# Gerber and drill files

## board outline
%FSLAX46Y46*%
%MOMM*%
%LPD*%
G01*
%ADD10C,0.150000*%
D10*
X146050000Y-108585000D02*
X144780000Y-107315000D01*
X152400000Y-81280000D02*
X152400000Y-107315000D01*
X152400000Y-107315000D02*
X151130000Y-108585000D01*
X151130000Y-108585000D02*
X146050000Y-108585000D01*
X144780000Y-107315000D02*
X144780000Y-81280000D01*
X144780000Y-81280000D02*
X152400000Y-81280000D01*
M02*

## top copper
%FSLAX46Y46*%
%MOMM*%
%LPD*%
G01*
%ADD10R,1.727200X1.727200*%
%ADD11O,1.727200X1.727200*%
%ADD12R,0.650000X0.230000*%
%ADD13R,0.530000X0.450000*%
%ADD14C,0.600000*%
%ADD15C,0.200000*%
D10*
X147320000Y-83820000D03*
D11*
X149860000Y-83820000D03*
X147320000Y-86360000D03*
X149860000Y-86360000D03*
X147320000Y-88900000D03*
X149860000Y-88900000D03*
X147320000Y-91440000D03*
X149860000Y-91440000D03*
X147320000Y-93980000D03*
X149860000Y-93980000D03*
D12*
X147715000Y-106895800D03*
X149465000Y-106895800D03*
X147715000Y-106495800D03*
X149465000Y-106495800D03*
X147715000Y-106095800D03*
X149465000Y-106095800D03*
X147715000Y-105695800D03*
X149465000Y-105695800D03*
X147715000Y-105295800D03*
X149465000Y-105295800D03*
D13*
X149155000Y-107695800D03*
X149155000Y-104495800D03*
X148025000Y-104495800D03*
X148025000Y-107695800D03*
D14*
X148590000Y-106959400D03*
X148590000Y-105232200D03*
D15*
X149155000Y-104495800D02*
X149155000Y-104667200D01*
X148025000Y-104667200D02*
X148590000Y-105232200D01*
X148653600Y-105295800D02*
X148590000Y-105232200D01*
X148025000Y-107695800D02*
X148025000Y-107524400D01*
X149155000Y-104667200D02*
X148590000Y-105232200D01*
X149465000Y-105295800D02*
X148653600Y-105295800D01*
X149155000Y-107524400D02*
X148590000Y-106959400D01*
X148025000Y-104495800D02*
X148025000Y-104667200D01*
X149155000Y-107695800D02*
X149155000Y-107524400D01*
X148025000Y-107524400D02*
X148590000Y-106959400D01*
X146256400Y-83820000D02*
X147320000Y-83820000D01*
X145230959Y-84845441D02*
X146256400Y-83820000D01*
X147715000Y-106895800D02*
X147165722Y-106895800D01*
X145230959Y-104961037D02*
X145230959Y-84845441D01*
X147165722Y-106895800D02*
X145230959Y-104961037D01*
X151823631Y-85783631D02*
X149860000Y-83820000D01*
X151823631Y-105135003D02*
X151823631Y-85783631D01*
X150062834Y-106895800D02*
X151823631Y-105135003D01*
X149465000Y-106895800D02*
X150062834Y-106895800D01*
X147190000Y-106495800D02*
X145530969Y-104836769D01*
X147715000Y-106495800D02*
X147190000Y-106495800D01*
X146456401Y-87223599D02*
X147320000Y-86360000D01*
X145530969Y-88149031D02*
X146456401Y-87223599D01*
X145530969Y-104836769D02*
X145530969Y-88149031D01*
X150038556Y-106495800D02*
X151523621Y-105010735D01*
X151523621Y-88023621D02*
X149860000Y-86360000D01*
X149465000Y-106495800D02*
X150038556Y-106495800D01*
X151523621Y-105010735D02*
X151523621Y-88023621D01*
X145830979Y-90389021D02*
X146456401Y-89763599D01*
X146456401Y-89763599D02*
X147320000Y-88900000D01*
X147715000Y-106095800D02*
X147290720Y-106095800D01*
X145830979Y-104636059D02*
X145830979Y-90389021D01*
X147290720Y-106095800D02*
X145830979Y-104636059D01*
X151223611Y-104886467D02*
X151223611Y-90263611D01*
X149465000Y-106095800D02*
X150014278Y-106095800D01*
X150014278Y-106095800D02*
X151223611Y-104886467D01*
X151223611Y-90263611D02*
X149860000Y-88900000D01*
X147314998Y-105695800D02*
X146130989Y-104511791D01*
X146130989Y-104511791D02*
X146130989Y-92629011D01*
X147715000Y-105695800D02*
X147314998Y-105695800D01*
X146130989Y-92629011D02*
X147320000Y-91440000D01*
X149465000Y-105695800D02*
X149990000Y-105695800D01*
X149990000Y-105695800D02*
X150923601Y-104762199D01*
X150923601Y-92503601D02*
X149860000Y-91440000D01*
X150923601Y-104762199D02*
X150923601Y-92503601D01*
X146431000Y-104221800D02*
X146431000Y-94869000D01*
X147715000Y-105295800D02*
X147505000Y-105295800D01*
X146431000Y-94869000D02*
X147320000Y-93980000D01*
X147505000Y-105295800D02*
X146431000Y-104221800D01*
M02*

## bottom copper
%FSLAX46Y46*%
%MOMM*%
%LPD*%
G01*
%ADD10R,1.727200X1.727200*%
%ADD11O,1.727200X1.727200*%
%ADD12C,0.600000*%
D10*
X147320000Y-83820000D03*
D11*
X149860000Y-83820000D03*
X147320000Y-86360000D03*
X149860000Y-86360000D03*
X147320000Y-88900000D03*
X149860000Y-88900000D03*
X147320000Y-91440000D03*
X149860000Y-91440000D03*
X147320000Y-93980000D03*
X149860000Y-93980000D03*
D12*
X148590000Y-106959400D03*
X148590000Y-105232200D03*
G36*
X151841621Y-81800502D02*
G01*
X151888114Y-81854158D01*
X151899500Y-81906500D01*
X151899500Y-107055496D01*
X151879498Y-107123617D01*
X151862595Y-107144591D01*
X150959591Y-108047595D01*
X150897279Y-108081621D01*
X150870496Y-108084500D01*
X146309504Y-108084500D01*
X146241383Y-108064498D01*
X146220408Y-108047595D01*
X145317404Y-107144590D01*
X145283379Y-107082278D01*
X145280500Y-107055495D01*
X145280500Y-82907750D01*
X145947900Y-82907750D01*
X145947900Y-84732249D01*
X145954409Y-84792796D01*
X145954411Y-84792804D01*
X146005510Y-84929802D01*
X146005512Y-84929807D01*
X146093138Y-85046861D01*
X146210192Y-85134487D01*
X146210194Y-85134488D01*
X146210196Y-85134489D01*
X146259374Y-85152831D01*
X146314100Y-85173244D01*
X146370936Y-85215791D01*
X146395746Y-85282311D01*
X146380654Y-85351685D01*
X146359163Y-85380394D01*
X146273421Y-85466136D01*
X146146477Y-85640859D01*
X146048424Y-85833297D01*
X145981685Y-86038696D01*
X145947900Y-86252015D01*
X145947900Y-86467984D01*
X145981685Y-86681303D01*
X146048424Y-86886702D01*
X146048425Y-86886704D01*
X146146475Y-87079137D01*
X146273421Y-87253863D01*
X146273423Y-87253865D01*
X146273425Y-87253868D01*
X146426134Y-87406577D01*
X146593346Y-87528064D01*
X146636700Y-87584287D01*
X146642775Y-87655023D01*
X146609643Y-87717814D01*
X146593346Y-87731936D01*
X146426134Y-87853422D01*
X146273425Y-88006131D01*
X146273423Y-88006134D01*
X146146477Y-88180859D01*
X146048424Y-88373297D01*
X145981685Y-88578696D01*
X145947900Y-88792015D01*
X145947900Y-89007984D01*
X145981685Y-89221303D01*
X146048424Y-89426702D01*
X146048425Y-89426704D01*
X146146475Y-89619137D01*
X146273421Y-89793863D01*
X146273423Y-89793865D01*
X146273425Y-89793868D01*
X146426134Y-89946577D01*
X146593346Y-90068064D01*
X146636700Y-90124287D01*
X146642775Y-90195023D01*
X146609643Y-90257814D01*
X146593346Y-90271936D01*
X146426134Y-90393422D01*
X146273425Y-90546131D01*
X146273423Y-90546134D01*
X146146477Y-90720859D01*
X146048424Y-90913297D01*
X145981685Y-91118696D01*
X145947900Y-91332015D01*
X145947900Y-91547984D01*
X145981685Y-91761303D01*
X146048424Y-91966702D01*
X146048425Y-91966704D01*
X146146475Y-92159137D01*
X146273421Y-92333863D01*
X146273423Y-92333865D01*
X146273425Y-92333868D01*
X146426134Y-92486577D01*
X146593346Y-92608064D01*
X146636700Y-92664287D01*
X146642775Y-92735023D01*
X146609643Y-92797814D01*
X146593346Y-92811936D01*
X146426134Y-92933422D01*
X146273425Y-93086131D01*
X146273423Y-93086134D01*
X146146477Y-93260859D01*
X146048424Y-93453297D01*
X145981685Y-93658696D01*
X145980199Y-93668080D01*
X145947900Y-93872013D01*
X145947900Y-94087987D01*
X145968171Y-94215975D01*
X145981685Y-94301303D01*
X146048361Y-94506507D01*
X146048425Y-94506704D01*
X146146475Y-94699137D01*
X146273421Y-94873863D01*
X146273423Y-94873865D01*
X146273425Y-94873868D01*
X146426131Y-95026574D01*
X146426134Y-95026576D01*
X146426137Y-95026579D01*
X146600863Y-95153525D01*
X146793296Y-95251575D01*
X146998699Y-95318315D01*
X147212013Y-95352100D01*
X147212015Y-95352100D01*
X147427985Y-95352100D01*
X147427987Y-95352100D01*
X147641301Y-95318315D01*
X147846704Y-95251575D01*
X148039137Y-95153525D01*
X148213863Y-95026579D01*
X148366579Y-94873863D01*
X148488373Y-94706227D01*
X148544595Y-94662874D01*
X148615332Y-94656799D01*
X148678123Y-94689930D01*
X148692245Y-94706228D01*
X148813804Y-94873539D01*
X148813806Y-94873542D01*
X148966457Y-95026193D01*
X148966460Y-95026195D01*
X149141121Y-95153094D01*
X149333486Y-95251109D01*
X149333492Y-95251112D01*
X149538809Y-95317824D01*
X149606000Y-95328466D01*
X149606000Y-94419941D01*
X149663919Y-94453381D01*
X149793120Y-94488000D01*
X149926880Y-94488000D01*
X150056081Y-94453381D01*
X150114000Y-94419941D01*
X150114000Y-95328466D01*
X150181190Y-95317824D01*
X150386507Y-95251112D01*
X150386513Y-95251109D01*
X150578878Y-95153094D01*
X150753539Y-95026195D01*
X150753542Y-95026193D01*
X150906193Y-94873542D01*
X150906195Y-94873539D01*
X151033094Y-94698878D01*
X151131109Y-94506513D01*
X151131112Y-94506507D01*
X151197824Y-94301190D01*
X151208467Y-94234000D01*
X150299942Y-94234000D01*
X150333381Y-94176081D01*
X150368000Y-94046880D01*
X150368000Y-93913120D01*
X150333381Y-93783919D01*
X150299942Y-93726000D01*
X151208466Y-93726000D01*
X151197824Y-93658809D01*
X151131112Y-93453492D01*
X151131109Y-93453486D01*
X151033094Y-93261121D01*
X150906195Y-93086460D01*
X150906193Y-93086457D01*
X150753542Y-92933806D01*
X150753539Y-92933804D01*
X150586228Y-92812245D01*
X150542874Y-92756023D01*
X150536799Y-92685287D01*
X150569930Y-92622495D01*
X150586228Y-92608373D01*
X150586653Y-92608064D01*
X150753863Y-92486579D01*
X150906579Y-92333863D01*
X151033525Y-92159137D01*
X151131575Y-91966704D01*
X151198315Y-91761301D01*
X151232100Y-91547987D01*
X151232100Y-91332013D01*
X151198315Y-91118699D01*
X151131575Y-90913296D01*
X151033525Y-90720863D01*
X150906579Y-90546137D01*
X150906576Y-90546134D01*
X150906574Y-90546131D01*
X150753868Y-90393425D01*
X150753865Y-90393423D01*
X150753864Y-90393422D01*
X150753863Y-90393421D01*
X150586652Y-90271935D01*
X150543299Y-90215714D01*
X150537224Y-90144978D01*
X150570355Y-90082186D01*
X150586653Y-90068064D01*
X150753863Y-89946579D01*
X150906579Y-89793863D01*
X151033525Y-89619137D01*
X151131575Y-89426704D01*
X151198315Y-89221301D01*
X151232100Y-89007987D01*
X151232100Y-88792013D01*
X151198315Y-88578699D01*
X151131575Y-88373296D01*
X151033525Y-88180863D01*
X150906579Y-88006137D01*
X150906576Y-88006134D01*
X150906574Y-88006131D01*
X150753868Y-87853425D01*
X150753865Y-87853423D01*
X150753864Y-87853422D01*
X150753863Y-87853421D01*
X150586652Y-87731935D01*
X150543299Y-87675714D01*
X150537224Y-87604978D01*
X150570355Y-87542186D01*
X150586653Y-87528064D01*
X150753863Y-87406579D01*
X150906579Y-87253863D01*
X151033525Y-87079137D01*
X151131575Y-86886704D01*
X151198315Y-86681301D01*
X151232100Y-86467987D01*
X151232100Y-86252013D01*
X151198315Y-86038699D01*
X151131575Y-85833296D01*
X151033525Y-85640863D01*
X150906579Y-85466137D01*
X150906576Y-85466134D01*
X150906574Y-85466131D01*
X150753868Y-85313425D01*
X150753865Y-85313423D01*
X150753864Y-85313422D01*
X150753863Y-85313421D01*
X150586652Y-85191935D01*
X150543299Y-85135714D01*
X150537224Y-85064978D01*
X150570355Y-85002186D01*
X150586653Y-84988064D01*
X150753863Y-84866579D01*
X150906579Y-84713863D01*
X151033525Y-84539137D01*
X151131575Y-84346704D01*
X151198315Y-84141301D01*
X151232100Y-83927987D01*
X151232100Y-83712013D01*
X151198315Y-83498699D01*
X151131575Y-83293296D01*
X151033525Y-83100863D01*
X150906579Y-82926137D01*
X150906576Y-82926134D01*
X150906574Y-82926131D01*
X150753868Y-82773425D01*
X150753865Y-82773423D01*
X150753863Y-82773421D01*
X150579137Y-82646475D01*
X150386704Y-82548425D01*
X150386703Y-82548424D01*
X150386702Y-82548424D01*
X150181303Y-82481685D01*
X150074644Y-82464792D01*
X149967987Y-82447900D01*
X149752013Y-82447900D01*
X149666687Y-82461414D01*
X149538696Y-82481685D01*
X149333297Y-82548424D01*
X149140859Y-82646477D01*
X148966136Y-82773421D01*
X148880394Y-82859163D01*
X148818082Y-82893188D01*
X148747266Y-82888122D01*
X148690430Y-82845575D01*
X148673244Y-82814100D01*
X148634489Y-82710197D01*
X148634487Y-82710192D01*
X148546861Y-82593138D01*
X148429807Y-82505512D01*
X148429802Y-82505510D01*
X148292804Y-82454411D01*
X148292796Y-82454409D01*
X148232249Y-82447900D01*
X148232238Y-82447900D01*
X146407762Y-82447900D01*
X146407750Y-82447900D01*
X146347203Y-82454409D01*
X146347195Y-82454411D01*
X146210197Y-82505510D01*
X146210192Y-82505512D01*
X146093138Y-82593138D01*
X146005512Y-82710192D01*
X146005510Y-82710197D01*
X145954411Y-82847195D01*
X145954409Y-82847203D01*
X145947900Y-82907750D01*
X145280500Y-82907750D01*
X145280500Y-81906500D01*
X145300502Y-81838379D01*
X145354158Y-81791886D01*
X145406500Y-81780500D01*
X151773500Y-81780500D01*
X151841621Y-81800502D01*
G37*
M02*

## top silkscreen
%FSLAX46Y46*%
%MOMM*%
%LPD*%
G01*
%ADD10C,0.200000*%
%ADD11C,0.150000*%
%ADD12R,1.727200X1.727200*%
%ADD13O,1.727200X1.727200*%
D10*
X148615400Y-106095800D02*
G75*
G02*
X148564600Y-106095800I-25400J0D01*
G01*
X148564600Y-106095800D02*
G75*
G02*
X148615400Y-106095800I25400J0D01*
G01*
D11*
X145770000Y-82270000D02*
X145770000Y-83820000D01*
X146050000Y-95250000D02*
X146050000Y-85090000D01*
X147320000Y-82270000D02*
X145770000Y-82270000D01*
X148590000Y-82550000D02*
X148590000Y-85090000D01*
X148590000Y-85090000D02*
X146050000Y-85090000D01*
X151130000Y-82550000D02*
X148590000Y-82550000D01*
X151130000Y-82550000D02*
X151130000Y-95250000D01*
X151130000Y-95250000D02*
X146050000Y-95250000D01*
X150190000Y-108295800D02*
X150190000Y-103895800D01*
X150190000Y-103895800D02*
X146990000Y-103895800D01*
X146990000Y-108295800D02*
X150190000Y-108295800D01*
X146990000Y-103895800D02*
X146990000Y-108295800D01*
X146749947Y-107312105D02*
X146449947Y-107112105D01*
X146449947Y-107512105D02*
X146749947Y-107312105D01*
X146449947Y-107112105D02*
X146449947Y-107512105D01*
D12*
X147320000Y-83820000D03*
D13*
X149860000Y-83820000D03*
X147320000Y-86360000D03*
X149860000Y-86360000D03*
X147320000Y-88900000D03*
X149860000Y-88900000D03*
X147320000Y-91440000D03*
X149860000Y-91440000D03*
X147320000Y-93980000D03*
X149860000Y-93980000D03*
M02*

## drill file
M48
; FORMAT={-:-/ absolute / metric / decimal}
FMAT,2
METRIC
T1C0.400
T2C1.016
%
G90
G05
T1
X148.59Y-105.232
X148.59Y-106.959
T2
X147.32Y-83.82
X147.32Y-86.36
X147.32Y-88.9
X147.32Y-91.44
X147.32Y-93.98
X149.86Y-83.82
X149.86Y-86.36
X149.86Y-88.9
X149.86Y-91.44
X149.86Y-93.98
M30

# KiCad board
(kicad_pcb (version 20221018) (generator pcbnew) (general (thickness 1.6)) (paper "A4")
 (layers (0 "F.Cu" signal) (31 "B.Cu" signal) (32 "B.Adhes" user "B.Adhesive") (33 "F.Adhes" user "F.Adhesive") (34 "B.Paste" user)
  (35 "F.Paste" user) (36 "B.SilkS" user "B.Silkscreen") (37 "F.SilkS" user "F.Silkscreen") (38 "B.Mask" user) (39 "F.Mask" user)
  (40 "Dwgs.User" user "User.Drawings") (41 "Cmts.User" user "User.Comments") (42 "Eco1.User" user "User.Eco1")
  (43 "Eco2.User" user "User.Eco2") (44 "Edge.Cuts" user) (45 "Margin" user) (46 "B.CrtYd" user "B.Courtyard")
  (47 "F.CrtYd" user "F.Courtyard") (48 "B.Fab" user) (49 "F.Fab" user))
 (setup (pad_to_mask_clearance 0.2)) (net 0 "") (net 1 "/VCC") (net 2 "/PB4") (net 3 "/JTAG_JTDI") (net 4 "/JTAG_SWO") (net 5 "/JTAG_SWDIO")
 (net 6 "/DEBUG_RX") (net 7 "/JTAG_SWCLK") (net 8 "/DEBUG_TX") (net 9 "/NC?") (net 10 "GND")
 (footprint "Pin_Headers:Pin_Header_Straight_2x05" (layer "F.Cu") (at 147.32 83.82)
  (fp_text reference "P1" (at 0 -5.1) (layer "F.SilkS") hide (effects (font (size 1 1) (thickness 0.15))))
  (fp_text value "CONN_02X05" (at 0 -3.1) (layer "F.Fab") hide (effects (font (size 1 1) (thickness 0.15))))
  (fp_line (start -1.55 -1.55) (end -1.55 0) (stroke (width 0.15) (type solid)) (layer "F.SilkS"))
  (fp_line (start -1.27 11.43) (end -1.27 1.27) (stroke (width 0.15) (type solid)) (layer "F.SilkS"))
  (fp_line (start 0 -1.55) (end -1.55 -1.55) (stroke (width 0.15) (type solid)) (layer "F.SilkS"))
  (fp_line (start 1.27 -1.27) (end 1.27 1.27) (stroke (width 0.15) (type solid)) (layer "F.SilkS"))
  (fp_line (start 1.27 1.27) (end -1.27 1.27) (stroke (width 0.15) (type solid)) (layer "F.SilkS"))
  (fp_line (start 3.81 -1.27) (end 1.27 -1.27) (stroke (width 0.15) (type solid)) (layer "F.SilkS"))
  (fp_line (start 3.81 -1.27) (end 3.81 11.43) (stroke (width 0.15) (type solid)) (layer "F.SilkS"))
  (fp_line (start 3.81 11.43) (end -1.27 11.43) (stroke (width 0.15) (type solid)) (layer "F.SilkS"))
  (pad "1" thru_hole rect (at 0 0) (size 1.7272 1.7272) (drill 1.016) (layers "*.Cu" "*.Mask" "F.SilkS") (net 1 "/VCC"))
  (pad "2" thru_hole oval (at 2.54 0) (size 1.7272 1.7272) (drill 1.016) (layers "*.Cu" "*.Mask" "F.SilkS") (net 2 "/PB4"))
  (pad "3" thru_hole oval (at 0 2.54) (size 1.7272 1.7272) (drill 1.016) (layers "*.Cu" "*.Mask" "F.SilkS") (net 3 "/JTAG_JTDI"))
  (pad "4" thru_hole oval (at 2.54 2.54) (size 1.7272 1.7272) (drill 1.016) (layers "*.Cu" "*.Mask" "F.SilkS") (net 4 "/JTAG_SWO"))
  (pad "5" thru_hole oval (at 0 5.08) (size 1.7272 1.7272) (drill 1.016) (layers "*.Cu" "*.Mask" "F.SilkS") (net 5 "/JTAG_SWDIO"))
  (pad "6" thru_hole oval (at 2.54 5.08) (size 1.7272 1.7272) (drill 1.016) (layers "*.Cu" "*.Mask" "F.SilkS") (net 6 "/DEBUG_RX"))
  (pad "7" thru_hole oval (at 0 7.62) (size 1.7272 1.7272) (drill 1.016) (layers "*.Cu" "*.Mask" "F.SilkS") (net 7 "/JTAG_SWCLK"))
  (pad "8" thru_hole oval (at 2.54 7.62) (size 1.7272 1.7272) (drill 1.016) (layers "*.Cu" "*.Mask" "F.SilkS") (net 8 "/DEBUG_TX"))
  (pad "9" thru_hole oval (at 0 10.16) (size 1.7272 1.7272) (drill 1.016) (layers "*.Cu" "*.Mask" "F.SilkS") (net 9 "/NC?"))
  (pad "10" thru_hole oval (at 2.54 10.16) (size 1.7272 1.7272) (drill 1.016) (layers "*.Cu" "*.Mask" "F.SilkS") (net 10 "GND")))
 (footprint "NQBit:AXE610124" (layer "F.Cu") (at 148.59 106.0958 180)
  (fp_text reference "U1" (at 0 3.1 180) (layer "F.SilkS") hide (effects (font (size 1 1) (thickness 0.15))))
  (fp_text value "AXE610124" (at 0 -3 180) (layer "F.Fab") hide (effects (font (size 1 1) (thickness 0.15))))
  (fp_line (start -1.6 -2.2) (end -1.6 2.2) (stroke (width 0.15) (type solid)) (layer "F.SilkS"))
  (fp_line (start -1.6 2.2) (end 1.6 2.2) (stroke (width 0.15) (type solid)) (layer "F.SilkS"))
  (fp_line (start 1.6 -2.2) (end -1.6 -2.2) (stroke (width 0.15) (type solid)) (layer "F.SilkS"))
  (fp_line (start 1.6 2.2) (end 1.6 -2.2) (stroke (width 0.15) (type solid)) (layer "F.SilkS"))
  (fp_line (start 1.840053 -1.216305) (end 2.140053 -1.016305) (stroke (width 0.15) (type solid)) (layer "F.SilkS"))
  (fp_line (start 2.140053 -1.416305) (end 1.840053 -1.216305) (stroke (width 0.15) (type solid)) (layer "F.SilkS"))
  (fp_line (start 2.140053 -1.016305) (end 2.140053 -1.416305) (stroke (width 0.15) (type solid)) (layer "F.SilkS"))
  (pad "1" smd rect (at 0.875 -0.8 180) (size 0.65 0.23) (layers "F.Cu" "F.Paste" "F.Mask") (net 1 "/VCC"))
  (pad "2" smd rect (at -0.875 -0.8 180) (size 0.65 0.23) (layers "F.Cu" "F.Paste" "F.Mask") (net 2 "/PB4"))
  (pad "3" smd rect (at 0.875 -0.4 180) (size 0.65 0.23) (layers "F.Cu" "F.Paste" "F.Mask") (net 3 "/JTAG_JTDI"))
  (pad "4" smd rect (at -0.875 -0.4 180) (size 0.65 0.23) (layers "F.Cu" "F.Paste" "F.Mask") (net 4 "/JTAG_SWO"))
  (pad "5" smd rect (at 0.875 0 180) (size 0.65 0.23) (layers "F.Cu" "F.Paste" "F.Mask") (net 5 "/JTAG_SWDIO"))
  (pad "6" smd rect (at -0.875 0 180) (size 0.65 0.23) (layers "F.Cu" "F.Paste" "F.Mask") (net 6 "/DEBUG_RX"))
  (pad "7" smd rect (at 0.875 0.4 180) (size 0.65 0.23) (layers "F.Cu" "F.Paste" "F.Mask") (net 7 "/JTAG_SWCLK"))
  (pad "8" smd rect (at -0.875 0.4 180) (size 0.65 0.23) (layers "F.Cu" "F.Paste" "F.Mask") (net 8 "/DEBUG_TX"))
  (pad "9" smd rect (at 0.875 0.8 180) (size 0.65 0.23) (layers "F.Cu" "F.Paste" "F.Mask") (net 9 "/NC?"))
  (pad "10" smd rect (at -0.875 0.8 180) (size 0.65 0.23) (layers "F.Cu" "F.Paste" "F.Mask") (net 10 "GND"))
  (pad "P1" smd rect (at -0.565 -1.6 180) (size 0.53 0.45) (layers "F.Cu" "F.Paste" "F.Mask") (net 10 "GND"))
  (pad "P2" smd rect (at -0.565 1.6 180) (size 0.53 0.45) (layers "F.Cu" "F.Paste" "F.Mask") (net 10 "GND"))
  (pad "P3" smd rect (at 0.565 1.6 180) (size 0.53 0.45) (layers "F.Cu" "F.Paste" "F.Mask") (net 10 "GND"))
  (pad "P4" smd rect (at 0.565 -1.6 180) (size 0.53 0.45) (layers "F.Cu" "F.Paste" "F.Mask") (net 10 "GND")))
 (gr_circle (center 148.59 106.0958) (end 148.6154 106.0958) (stroke (width 0.2) (type solid)) (fill none) (layer "F.SilkS"))
 (gr_line (start 146.05 108.585) (end 144.78 107.315) (stroke (width 0.15) (type solid)) (layer "Edge.Cuts"))
 (gr_line (start 152.4 81.28) (end 152.4 107.315) (stroke (width 0.15) (type solid)) (layer "Edge.Cuts"))
 (gr_line (start 152.4 107.315) (end 151.13 108.585) (stroke (width 0.15) (type solid)) (layer "Edge.Cuts"))
 (gr_line (start 151.13 108.585) (end 146.05 108.585) (stroke (width 0.15) (type solid)) (layer "Edge.Cuts"))
 (gr_line (start 144.78 107.315) (end 144.78 81.28) (stroke (width 0.15) (type solid)) (layer "Edge.Cuts"))
 (gr_line (start 144.78 81.28) (end 152.4 81.28) (stroke (width 0.15) (type solid)) (layer "Edge.Cuts"))
 (segment (start 149.155 104.4958) (end 149.155 104.6672) (width 0.2) (layer "F.Cu") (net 10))
 (segment (start 148.025 104.6672) (end 148.59 105.2322) (width 0.2) (layer "F.Cu") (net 10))
 (segment (start 148.6536 105.2958) (end 148.59 105.2322) (width 0.2) (layer "F.Cu") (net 10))
 (segment (start 148.025 107.6958) (end 148.025 107.5244) (width 0.2) (layer "F.Cu") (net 10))
 (segment (start 149.155 104.6672) (end 148.59 105.2322) (width 0.2) (layer "F.Cu") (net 10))
 (segment (start 149.465 105.2958) (end 148.6536 105.2958) (width 0.2) (layer "F.Cu") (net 10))
 (segment (start 149.155 107.5244) (end 148.59 106.9594) (width 0.2) (layer "F.Cu") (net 10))
 (segment (start 148.025 104.4958) (end 148.025 104.6672) (width 0.2) (layer "F.Cu") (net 10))
 (segment (start 149.155 107.6958) (end 149.155 107.5244) (width 0.2) (layer "F.Cu") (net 10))
 (segment (start 148.025 107.5244) (end 148.59 106.9594) (width 0.2) (layer "F.Cu") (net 10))
 (via (at 148.59 106.9594) (size 0.6) (drill 0.4) (layers "F.Cu" "B.Cu") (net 10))
 (via (at 148.59 105.2322) (size 0.6) (drill 0.4) (layers "F.Cu" "B.Cu") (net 10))
 (segment (start 146.2564 83.82) (end 147.32 83.82) (width 0.2) (layer "F.Cu") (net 1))
 (segment (start 145.230959 84.845441) (end 146.2564 83.82) (width 0.2) (layer "F.Cu") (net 1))
 (segment (start 147.715 106.8958) (end 147.165722 106.8958) (width 0.2) (layer "F.Cu") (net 1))
 (segment (start 145.230959 104.961037) (end 145.230959 84.845441) (width 0.2) (layer "F.Cu") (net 1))
 (segment (start 147.165722 106.8958) (end 145.230959 104.961037) (width 0.2) (layer "F.Cu") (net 1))
 (segment (start 151.823631 85.783631) (end 149.86 83.82) (width 0.2) (layer "F.Cu") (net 2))
 (segment (start 151.823631 105.135003) (end 151.823631 85.783631) (width 0.2) (layer "F.Cu") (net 2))
 (segment (start 150.062834 106.8958) (end 151.823631 105.135003) (width 0.2) (layer "F.Cu") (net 2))
 (segment (start 149.465 106.8958) (end 150.062834 106.8958) (width 0.2) (layer "F.Cu") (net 2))
 (segment (start 147.19 106.4958) (end 145.530969 104.836769) (width 0.2) (layer "F.Cu") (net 3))
 (segment (start 147.715 106.4958) (end 147.19 106.4958) (width 0.2) (layer "F.Cu") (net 3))
 (segment (start 146.456401 87.223599) (end 147.32 86.36) (width 0.2) (layer "F.Cu") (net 3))
 (segment (start 145.530969 88.149031) (end 146.456401 87.223599) (width 0.2) (layer "F.Cu") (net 3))
 (segment (start 145.530969 104.836769) (end 145.530969 88.149031) (width 0.2) (layer "F.Cu") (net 3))
 (segment (start 150.038556 106.4958) (end 151.523621 105.010735) (width 0.2) (layer "F.Cu") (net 4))
 (segment (start 151.523621 88.023621) (end 149.86 86.36) (width 0.2) (layer "F.Cu") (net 4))
 (segment (start 149.465 106.4958) (end 150.038556 106.4958) (width 0.2) (layer "F.Cu") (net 4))
 (segment (start 151.523621 105.010735) (end 151.523621 88.023621) (width 0.2) (layer "F.Cu") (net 4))
 (segment (start 145.830979 90.389021) (end 146.456401 89.763599) (width 0.2) (layer "F.Cu") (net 5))
 (segment (start 146.456401 89.763599) (end 147.32 88.9) (width 0.2) (layer "F.Cu") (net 5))
 (segment (start 147.715 106.0958) (end 147.29072 106.0958) (width 0.2) (layer "F.Cu") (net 5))
 (segment (start 145.830979 104.636059) (end 145.830979 90.389021) (width 0.2) (layer "F.Cu") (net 5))
 (segment (start 147.29072 106.0958) (end 145.830979 104.636059) (width 0.2) (layer "F.Cu") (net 5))
 (segment (start 151.223611 104.886467) (end 151.223611 90.263611) (width 0.2) (layer "F.Cu") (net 6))
 (segment (start 149.465 106.0958) (end 150.014278 106.0958) (width 0.2) (layer "F.Cu") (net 6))
 (segment (start 150.014278 106.0958) (end 151.223611 104.886467) (width 0.2) (layer "F.Cu") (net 6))
 (segment (start 151.223611 90.263611) (end 149.86 88.9) (width 0.2) (layer "F.Cu") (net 6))
 (segment (start 147.314998 105.6958) (end 146.130989 104.511791) (width 0.2) (layer "F.Cu") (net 7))
 (segment (start 146.130989 104.511791) (end 146.130989 92.629011) (width 0.2) (layer "F.Cu") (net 7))
 (segment (start 147.715 105.6958) (end 147.314998 105.6958) (width 0.2) (layer "F.Cu") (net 7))
 (segment (start 146.130989 92.629011) (end 147.32 91.44) (width 0.2) (layer "F.Cu") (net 7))
 (segment (start 149.465 105.6958) (end 149.99 105.6958) (width 0.2) (layer "F.Cu") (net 8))
 (segment (start 149.99 105.6958) (end 150.923601 104.762199) (width 0.2) (layer "F.Cu") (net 8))
 (segment (start 150.923601 92.503601) (end 149.86 91.44) (width 0.2) (layer "F.Cu") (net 8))
 (segment (start 150.923601 104.762199) (end 150.923601 92.503601) (width 0.2) (layer "F.Cu") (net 8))
 (segment (start 146.431 104.2218) (end 146.431 94.869) (width 0.2) (layer "F.Cu") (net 9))
 (segment (start 147.715 105.2958) (end 147.505 105.2958) (width 0.2) (layer "F.Cu") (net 9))
 (segment (start 146.431 94.869) (end 147.32 93.98) (width 0.2) (layer "F.Cu") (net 9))
 (segment (start 147.505 105.2958) (end 146.431 104.2218) (width 0.2) (layer "F.Cu") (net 9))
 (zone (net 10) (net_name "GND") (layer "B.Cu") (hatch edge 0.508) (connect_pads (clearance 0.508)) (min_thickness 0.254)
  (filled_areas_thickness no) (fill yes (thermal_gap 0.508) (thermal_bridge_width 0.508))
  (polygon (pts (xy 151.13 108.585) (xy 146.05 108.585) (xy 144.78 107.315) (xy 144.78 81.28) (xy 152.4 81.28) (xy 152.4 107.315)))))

